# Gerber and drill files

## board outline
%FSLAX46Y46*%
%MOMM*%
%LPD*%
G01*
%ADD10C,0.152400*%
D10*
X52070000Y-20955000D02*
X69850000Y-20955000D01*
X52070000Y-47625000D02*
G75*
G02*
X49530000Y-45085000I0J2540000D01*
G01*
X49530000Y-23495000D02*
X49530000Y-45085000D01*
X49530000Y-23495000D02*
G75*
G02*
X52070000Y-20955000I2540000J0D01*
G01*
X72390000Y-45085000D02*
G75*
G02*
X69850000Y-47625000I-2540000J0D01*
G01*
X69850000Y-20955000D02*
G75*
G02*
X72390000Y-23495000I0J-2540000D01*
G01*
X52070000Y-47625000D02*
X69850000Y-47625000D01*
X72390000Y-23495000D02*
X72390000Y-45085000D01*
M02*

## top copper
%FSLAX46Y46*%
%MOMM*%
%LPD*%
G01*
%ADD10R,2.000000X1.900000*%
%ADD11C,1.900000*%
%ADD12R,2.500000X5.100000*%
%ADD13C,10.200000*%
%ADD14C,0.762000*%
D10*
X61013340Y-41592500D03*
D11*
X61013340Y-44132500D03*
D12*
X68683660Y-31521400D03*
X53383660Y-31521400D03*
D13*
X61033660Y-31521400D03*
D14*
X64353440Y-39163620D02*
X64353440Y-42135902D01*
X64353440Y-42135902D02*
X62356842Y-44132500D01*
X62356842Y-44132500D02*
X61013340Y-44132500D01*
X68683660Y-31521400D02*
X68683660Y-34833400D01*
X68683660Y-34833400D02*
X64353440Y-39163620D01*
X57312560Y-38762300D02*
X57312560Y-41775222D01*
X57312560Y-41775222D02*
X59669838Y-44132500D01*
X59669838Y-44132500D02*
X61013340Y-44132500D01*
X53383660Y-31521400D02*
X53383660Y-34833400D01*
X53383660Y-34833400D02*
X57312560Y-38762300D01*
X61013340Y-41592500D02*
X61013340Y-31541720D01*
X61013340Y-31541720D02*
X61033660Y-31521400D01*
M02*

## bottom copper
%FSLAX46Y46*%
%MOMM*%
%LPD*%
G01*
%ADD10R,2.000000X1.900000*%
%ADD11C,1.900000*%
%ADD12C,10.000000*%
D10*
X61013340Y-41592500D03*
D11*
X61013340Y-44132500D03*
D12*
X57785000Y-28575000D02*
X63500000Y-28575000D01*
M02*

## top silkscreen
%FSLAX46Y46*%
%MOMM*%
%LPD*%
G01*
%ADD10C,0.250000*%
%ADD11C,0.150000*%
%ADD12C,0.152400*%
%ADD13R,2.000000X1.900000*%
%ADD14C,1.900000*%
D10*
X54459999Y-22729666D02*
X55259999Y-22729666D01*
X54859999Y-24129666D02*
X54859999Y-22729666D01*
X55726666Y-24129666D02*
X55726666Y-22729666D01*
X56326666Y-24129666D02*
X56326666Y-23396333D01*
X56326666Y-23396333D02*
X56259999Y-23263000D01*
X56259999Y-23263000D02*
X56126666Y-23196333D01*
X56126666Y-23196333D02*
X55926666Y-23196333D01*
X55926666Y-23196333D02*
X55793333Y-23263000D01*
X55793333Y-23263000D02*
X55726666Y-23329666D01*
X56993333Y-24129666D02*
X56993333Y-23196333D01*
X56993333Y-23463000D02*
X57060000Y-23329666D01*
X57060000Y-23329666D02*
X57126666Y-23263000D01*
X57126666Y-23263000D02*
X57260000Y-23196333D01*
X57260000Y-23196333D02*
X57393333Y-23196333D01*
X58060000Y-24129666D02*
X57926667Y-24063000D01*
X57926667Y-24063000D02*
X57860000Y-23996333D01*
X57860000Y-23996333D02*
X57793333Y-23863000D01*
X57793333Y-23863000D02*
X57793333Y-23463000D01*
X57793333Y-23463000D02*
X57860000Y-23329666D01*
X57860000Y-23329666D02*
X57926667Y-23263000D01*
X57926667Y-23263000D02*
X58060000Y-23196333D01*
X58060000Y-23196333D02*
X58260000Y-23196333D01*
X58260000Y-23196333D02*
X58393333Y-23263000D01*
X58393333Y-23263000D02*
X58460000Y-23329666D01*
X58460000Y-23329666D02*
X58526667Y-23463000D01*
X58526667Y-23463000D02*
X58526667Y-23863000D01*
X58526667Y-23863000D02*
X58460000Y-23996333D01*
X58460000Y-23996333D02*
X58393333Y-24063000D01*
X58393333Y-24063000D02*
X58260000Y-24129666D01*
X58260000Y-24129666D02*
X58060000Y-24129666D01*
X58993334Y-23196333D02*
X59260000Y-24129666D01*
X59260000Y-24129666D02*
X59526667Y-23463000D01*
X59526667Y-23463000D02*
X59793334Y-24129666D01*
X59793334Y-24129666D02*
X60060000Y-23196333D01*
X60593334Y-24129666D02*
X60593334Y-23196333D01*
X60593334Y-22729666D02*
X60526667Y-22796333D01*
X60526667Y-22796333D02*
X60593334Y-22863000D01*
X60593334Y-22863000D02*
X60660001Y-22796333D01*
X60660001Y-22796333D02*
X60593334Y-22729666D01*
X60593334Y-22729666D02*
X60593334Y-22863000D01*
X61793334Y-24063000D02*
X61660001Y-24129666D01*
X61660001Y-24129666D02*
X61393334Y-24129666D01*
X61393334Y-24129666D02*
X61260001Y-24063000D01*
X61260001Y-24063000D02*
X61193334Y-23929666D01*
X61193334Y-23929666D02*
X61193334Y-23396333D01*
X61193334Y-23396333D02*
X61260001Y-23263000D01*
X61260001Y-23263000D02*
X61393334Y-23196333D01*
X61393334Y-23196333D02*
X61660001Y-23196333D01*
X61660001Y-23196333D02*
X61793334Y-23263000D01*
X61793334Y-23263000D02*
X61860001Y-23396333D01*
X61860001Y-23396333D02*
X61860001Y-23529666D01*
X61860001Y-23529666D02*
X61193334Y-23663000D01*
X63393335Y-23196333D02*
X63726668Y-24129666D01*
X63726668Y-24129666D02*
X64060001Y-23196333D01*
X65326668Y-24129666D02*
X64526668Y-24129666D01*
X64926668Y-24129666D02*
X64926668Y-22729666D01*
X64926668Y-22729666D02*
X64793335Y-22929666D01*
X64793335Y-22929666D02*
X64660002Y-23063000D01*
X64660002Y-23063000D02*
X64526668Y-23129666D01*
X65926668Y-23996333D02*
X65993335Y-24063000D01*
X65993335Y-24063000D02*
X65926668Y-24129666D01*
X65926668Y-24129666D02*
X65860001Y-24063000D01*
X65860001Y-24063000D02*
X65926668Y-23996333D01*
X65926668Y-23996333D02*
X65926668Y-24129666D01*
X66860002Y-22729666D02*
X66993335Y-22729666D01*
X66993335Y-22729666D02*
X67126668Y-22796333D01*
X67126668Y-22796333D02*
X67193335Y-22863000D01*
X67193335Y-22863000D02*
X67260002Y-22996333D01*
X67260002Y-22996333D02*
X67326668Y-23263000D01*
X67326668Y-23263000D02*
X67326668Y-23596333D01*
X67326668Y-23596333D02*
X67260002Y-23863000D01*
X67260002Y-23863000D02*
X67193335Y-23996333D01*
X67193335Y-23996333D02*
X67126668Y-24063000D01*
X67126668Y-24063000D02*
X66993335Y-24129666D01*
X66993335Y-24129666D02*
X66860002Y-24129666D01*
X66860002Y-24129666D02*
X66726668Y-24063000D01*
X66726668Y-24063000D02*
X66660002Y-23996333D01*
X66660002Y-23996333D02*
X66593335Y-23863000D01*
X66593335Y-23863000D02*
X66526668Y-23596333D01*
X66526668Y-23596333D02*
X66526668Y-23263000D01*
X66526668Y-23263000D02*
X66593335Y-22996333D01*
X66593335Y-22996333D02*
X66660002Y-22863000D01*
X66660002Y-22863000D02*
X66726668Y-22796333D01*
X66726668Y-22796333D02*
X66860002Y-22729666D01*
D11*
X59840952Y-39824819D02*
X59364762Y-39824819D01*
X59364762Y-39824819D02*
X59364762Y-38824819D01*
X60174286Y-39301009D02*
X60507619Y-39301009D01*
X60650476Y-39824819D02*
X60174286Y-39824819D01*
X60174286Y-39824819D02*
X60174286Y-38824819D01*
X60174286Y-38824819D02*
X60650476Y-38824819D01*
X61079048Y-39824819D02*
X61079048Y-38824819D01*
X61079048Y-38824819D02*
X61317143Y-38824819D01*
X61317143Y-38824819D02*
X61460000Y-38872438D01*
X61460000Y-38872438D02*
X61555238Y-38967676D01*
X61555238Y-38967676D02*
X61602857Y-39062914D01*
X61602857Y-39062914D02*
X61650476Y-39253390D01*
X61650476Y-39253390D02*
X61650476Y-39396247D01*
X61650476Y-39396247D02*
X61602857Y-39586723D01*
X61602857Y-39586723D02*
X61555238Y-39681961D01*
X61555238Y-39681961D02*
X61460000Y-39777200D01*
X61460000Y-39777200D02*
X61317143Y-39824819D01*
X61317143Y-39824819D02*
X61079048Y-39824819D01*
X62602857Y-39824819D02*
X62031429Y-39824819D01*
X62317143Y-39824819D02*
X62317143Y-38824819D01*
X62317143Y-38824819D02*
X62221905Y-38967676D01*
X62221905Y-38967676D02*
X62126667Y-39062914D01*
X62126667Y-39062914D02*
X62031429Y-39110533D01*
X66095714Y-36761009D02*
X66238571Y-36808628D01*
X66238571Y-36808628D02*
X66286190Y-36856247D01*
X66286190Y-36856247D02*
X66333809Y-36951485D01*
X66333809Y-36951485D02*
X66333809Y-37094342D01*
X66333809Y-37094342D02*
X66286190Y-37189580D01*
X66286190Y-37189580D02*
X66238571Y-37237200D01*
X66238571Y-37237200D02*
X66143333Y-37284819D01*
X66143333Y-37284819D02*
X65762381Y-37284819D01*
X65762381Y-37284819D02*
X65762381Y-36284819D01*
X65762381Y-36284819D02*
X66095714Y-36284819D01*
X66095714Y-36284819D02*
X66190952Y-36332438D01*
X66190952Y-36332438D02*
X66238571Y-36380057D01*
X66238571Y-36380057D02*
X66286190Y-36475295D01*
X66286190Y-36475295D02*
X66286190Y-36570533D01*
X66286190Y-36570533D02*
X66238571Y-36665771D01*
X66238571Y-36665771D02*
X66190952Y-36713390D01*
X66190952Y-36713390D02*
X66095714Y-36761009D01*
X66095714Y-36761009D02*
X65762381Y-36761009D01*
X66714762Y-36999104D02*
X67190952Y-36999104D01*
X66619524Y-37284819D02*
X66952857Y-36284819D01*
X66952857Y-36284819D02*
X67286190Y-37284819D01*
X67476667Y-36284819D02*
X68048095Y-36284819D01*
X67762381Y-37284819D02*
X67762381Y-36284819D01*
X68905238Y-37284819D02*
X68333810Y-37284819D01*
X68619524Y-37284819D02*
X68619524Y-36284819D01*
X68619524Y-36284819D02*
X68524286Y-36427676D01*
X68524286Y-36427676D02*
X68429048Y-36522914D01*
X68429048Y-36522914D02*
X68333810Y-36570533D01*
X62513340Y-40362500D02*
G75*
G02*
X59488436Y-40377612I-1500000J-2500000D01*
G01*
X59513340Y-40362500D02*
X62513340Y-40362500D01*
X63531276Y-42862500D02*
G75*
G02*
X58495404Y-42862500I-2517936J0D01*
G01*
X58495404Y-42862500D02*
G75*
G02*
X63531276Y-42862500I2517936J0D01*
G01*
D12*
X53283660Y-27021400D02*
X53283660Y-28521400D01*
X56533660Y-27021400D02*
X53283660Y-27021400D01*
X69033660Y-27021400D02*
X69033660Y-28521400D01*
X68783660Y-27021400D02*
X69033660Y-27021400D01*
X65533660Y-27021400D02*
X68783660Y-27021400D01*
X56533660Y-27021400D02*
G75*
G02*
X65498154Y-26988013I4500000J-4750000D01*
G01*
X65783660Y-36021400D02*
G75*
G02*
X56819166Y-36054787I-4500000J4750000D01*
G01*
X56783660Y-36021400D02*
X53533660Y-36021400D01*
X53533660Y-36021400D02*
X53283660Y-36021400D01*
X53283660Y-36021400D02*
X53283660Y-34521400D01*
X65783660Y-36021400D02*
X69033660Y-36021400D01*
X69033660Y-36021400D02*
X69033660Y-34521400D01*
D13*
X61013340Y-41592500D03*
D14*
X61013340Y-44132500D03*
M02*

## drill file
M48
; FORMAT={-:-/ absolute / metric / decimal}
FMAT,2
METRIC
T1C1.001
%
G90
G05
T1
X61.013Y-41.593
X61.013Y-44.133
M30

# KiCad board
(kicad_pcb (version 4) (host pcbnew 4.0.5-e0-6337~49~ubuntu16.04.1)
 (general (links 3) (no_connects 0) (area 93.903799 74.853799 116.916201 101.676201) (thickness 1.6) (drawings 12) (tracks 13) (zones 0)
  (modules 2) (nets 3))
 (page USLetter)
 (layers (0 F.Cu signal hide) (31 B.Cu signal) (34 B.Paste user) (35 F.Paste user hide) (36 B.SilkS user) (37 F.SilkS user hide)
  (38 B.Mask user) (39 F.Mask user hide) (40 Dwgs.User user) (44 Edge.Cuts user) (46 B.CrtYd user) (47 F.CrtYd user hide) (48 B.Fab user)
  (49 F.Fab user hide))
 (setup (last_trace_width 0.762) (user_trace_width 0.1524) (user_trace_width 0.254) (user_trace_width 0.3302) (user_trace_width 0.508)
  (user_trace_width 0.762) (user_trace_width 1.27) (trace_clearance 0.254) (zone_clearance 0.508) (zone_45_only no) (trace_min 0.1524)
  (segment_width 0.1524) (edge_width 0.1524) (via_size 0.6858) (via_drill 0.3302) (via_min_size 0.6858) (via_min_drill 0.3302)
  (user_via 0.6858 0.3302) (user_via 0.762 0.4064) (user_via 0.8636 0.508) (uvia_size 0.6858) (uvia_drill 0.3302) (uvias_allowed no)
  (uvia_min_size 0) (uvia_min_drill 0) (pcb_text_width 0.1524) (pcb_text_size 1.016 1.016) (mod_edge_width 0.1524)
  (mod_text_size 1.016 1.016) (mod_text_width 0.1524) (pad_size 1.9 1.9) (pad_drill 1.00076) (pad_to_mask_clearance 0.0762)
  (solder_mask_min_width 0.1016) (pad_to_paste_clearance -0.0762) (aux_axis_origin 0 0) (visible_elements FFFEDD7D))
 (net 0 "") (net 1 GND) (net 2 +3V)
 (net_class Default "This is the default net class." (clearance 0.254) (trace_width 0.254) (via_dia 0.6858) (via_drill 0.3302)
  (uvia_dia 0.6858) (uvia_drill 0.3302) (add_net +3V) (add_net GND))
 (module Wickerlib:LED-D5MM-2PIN (layer F.Cu) (at 61.01334 41.5925 270)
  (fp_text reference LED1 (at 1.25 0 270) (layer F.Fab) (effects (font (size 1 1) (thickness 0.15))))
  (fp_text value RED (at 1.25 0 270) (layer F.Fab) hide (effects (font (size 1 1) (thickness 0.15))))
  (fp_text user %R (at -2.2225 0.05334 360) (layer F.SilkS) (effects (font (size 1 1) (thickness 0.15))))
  (fp_arc (start 1.27 0) (end -1.23 -1.5) (angle 297.5) (layer F.SilkS) (width 0.15))
  (fp_line (start -1.23 1.5) (end -1.23 -1.5) (layer F.SilkS) (width 0.15))
  (fp_circle (center 1.27 0) (end 0.97 -2.5) (layer F.SilkS) (width 0.15))
  (pad 1 thru_hole rect (at 0 0) (size 2 1.9) (drill 1.00076) (layers *.Cu F.SilkS B.Mask) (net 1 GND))
  (pad 2 thru_hole circle (at 2.54 0 270) (size 1.9 1.9) (drill 1.00076) (layers *.Cu F.SilkS B.Mask) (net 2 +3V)))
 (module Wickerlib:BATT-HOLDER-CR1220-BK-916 (layer F.Cu) (at 61.03366 31.5214)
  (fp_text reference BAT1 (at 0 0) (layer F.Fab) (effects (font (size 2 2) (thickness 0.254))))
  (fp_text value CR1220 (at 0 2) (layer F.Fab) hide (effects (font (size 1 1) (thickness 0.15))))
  (fp_line (start -7.75 -4.5) (end -7.75 -3) (layer F.SilkS) (width 0.1524))
  (fp_line (start -4.5 -4.5) (end -7.75 -4.5) (layer F.SilkS) (width 0.1524))
  (fp_line (start 8 -4.5) (end 8 -3) (layer F.SilkS) (width 0.1524))
  (fp_line (start 7.75 -4.5) (end 8 -4.5) (layer F.SilkS) (width 0.1524))
  (fp_line (start 4.5 -4.5) (end 7.75 -4.5) (layer F.SilkS) (width 0.1524))
  (fp_arc (start 0 0.25) (end -4.5 -4.5) (angle 86.47690829) (layer F.SilkS) (width 0.1524))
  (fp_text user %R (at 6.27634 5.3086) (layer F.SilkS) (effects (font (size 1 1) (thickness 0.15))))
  (fp_arc (start 0.25 -0.25) (end 4.75 4.5) (angle 86.47690829) (layer F.SilkS) (width 0.1524))
  (fp_line (start -4.25 4.5) (end -7.5 4.5) (layer F.SilkS) (width 0.1524))
  (fp_line (start -7.5 4.5) (end -7.75 4.5) (layer F.SilkS) (width 0.1524))
  (fp_line (start -7.75 4.5) (end -7.75 3) (layer F.SilkS) (width 0.1524))
  (fp_line (start 4.75 4.5) (end 8 4.5) (layer F.SilkS) (width 0.1524))
  (fp_line (start 8 4.5) (end 8 3) (layer F.SilkS) (width 0.1524))
  (pad 1 smd rect (at 7.65 0) (size 2.5 5.1) (layers F.Cu F.Paste F.Mask) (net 2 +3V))
  (pad 1 smd rect (at -7.65 0) (size 2.5 5.1) (layers F.Cu F.Paste F.Mask) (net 2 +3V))
  (pad GND smd circle (at 0 0) (size 10.2 10.2) (layers F.Cu F.Mask) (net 1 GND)))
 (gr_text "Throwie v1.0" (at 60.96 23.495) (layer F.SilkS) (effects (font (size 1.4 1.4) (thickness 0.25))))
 (gr_line (start 52.07 20.955) (end 69.85 20.955) (layer Edge.Cuts) (width 0.1524))
 (gr_arc (start 52.07 45.085) (end 52.07 47.625) (angle 90) (layer Edge.Cuts) (width 0.1524))
 (gr_line (start 49.53 23.495) (end 49.53 45.085) (layer Edge.Cuts) (width 0.1524))
 (gr_arc (start 52.07 23.495) (end 49.53 23.495) (angle 90) (layer Edge.Cuts) (width 0.1524))
 (gr_arc (start 69.85 45.085) (end 72.39 45.085) (angle 90) (layer Edge.Cuts) (width 0.1524))
 (gr_arc (start 69.85 23.495) (end 69.85 20.955) (angle 90) (layer Edge.Cuts) (width 0.1524))
 (gr_line (start 52.07 47.625) (end 69.85 47.625) (layer Edge.Cuts) (width 0.1524))
 (gr_line (start 72.39 23.495) (end 72.39 45.085) (layer Edge.Cuts) (width 0.1524))
 (segment (start 57.785 28.575) (end 63.5 28.575) (width 10) (layer B.Cu) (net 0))
 (segment (start 64.35344 39.16362) (end 64.35344 42.135902) (width 0.762) (layer F.Cu) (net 2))
 (segment (start 64.35344 42.135902) (end 62.356842 44.1325) (width 0.762) (layer F.Cu) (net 2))
 (segment (start 62.356842 44.1325) (end 61.01334 44.1325) (width 0.762) (layer F.Cu) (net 2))
 (segment (start 68.68366 31.5214) (end 68.68366 34.8334) (width 0.762) (layer F.Cu) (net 2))
 (segment (start 68.68366 34.8334) (end 64.35344 39.16362) (width 0.762) (layer F.Cu) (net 2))
 (segment (start 57.31256 38.7623) (end 57.31256 41.775222) (width 0.762) (layer F.Cu) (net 2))
 (segment (start 57.31256 41.775222) (end 59.669838 44.1325) (width 0.762) (layer F.Cu) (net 2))
 (segment (start 59.669838 44.1325) (end 61.01334 44.1325) (width 0.762) (layer F.Cu) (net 2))
 (segment (start 53.38366 31.5214) (end 53.38366 34.8334) (width 0.762) (layer F.Cu) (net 2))
 (segment (start 53.38366 34.8334) (end 57.31256 38.7623) (width 0.762) (layer F.Cu) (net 2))
 (segment (start 61.01334 41.5925) (end 61.01334 31.54172) (width 0.762) (layer F.Cu) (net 1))
 (segment (start 61.01334 31.54172) (end 61.03366 31.5214) (width 0.762) (layer F.Cu) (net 1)))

